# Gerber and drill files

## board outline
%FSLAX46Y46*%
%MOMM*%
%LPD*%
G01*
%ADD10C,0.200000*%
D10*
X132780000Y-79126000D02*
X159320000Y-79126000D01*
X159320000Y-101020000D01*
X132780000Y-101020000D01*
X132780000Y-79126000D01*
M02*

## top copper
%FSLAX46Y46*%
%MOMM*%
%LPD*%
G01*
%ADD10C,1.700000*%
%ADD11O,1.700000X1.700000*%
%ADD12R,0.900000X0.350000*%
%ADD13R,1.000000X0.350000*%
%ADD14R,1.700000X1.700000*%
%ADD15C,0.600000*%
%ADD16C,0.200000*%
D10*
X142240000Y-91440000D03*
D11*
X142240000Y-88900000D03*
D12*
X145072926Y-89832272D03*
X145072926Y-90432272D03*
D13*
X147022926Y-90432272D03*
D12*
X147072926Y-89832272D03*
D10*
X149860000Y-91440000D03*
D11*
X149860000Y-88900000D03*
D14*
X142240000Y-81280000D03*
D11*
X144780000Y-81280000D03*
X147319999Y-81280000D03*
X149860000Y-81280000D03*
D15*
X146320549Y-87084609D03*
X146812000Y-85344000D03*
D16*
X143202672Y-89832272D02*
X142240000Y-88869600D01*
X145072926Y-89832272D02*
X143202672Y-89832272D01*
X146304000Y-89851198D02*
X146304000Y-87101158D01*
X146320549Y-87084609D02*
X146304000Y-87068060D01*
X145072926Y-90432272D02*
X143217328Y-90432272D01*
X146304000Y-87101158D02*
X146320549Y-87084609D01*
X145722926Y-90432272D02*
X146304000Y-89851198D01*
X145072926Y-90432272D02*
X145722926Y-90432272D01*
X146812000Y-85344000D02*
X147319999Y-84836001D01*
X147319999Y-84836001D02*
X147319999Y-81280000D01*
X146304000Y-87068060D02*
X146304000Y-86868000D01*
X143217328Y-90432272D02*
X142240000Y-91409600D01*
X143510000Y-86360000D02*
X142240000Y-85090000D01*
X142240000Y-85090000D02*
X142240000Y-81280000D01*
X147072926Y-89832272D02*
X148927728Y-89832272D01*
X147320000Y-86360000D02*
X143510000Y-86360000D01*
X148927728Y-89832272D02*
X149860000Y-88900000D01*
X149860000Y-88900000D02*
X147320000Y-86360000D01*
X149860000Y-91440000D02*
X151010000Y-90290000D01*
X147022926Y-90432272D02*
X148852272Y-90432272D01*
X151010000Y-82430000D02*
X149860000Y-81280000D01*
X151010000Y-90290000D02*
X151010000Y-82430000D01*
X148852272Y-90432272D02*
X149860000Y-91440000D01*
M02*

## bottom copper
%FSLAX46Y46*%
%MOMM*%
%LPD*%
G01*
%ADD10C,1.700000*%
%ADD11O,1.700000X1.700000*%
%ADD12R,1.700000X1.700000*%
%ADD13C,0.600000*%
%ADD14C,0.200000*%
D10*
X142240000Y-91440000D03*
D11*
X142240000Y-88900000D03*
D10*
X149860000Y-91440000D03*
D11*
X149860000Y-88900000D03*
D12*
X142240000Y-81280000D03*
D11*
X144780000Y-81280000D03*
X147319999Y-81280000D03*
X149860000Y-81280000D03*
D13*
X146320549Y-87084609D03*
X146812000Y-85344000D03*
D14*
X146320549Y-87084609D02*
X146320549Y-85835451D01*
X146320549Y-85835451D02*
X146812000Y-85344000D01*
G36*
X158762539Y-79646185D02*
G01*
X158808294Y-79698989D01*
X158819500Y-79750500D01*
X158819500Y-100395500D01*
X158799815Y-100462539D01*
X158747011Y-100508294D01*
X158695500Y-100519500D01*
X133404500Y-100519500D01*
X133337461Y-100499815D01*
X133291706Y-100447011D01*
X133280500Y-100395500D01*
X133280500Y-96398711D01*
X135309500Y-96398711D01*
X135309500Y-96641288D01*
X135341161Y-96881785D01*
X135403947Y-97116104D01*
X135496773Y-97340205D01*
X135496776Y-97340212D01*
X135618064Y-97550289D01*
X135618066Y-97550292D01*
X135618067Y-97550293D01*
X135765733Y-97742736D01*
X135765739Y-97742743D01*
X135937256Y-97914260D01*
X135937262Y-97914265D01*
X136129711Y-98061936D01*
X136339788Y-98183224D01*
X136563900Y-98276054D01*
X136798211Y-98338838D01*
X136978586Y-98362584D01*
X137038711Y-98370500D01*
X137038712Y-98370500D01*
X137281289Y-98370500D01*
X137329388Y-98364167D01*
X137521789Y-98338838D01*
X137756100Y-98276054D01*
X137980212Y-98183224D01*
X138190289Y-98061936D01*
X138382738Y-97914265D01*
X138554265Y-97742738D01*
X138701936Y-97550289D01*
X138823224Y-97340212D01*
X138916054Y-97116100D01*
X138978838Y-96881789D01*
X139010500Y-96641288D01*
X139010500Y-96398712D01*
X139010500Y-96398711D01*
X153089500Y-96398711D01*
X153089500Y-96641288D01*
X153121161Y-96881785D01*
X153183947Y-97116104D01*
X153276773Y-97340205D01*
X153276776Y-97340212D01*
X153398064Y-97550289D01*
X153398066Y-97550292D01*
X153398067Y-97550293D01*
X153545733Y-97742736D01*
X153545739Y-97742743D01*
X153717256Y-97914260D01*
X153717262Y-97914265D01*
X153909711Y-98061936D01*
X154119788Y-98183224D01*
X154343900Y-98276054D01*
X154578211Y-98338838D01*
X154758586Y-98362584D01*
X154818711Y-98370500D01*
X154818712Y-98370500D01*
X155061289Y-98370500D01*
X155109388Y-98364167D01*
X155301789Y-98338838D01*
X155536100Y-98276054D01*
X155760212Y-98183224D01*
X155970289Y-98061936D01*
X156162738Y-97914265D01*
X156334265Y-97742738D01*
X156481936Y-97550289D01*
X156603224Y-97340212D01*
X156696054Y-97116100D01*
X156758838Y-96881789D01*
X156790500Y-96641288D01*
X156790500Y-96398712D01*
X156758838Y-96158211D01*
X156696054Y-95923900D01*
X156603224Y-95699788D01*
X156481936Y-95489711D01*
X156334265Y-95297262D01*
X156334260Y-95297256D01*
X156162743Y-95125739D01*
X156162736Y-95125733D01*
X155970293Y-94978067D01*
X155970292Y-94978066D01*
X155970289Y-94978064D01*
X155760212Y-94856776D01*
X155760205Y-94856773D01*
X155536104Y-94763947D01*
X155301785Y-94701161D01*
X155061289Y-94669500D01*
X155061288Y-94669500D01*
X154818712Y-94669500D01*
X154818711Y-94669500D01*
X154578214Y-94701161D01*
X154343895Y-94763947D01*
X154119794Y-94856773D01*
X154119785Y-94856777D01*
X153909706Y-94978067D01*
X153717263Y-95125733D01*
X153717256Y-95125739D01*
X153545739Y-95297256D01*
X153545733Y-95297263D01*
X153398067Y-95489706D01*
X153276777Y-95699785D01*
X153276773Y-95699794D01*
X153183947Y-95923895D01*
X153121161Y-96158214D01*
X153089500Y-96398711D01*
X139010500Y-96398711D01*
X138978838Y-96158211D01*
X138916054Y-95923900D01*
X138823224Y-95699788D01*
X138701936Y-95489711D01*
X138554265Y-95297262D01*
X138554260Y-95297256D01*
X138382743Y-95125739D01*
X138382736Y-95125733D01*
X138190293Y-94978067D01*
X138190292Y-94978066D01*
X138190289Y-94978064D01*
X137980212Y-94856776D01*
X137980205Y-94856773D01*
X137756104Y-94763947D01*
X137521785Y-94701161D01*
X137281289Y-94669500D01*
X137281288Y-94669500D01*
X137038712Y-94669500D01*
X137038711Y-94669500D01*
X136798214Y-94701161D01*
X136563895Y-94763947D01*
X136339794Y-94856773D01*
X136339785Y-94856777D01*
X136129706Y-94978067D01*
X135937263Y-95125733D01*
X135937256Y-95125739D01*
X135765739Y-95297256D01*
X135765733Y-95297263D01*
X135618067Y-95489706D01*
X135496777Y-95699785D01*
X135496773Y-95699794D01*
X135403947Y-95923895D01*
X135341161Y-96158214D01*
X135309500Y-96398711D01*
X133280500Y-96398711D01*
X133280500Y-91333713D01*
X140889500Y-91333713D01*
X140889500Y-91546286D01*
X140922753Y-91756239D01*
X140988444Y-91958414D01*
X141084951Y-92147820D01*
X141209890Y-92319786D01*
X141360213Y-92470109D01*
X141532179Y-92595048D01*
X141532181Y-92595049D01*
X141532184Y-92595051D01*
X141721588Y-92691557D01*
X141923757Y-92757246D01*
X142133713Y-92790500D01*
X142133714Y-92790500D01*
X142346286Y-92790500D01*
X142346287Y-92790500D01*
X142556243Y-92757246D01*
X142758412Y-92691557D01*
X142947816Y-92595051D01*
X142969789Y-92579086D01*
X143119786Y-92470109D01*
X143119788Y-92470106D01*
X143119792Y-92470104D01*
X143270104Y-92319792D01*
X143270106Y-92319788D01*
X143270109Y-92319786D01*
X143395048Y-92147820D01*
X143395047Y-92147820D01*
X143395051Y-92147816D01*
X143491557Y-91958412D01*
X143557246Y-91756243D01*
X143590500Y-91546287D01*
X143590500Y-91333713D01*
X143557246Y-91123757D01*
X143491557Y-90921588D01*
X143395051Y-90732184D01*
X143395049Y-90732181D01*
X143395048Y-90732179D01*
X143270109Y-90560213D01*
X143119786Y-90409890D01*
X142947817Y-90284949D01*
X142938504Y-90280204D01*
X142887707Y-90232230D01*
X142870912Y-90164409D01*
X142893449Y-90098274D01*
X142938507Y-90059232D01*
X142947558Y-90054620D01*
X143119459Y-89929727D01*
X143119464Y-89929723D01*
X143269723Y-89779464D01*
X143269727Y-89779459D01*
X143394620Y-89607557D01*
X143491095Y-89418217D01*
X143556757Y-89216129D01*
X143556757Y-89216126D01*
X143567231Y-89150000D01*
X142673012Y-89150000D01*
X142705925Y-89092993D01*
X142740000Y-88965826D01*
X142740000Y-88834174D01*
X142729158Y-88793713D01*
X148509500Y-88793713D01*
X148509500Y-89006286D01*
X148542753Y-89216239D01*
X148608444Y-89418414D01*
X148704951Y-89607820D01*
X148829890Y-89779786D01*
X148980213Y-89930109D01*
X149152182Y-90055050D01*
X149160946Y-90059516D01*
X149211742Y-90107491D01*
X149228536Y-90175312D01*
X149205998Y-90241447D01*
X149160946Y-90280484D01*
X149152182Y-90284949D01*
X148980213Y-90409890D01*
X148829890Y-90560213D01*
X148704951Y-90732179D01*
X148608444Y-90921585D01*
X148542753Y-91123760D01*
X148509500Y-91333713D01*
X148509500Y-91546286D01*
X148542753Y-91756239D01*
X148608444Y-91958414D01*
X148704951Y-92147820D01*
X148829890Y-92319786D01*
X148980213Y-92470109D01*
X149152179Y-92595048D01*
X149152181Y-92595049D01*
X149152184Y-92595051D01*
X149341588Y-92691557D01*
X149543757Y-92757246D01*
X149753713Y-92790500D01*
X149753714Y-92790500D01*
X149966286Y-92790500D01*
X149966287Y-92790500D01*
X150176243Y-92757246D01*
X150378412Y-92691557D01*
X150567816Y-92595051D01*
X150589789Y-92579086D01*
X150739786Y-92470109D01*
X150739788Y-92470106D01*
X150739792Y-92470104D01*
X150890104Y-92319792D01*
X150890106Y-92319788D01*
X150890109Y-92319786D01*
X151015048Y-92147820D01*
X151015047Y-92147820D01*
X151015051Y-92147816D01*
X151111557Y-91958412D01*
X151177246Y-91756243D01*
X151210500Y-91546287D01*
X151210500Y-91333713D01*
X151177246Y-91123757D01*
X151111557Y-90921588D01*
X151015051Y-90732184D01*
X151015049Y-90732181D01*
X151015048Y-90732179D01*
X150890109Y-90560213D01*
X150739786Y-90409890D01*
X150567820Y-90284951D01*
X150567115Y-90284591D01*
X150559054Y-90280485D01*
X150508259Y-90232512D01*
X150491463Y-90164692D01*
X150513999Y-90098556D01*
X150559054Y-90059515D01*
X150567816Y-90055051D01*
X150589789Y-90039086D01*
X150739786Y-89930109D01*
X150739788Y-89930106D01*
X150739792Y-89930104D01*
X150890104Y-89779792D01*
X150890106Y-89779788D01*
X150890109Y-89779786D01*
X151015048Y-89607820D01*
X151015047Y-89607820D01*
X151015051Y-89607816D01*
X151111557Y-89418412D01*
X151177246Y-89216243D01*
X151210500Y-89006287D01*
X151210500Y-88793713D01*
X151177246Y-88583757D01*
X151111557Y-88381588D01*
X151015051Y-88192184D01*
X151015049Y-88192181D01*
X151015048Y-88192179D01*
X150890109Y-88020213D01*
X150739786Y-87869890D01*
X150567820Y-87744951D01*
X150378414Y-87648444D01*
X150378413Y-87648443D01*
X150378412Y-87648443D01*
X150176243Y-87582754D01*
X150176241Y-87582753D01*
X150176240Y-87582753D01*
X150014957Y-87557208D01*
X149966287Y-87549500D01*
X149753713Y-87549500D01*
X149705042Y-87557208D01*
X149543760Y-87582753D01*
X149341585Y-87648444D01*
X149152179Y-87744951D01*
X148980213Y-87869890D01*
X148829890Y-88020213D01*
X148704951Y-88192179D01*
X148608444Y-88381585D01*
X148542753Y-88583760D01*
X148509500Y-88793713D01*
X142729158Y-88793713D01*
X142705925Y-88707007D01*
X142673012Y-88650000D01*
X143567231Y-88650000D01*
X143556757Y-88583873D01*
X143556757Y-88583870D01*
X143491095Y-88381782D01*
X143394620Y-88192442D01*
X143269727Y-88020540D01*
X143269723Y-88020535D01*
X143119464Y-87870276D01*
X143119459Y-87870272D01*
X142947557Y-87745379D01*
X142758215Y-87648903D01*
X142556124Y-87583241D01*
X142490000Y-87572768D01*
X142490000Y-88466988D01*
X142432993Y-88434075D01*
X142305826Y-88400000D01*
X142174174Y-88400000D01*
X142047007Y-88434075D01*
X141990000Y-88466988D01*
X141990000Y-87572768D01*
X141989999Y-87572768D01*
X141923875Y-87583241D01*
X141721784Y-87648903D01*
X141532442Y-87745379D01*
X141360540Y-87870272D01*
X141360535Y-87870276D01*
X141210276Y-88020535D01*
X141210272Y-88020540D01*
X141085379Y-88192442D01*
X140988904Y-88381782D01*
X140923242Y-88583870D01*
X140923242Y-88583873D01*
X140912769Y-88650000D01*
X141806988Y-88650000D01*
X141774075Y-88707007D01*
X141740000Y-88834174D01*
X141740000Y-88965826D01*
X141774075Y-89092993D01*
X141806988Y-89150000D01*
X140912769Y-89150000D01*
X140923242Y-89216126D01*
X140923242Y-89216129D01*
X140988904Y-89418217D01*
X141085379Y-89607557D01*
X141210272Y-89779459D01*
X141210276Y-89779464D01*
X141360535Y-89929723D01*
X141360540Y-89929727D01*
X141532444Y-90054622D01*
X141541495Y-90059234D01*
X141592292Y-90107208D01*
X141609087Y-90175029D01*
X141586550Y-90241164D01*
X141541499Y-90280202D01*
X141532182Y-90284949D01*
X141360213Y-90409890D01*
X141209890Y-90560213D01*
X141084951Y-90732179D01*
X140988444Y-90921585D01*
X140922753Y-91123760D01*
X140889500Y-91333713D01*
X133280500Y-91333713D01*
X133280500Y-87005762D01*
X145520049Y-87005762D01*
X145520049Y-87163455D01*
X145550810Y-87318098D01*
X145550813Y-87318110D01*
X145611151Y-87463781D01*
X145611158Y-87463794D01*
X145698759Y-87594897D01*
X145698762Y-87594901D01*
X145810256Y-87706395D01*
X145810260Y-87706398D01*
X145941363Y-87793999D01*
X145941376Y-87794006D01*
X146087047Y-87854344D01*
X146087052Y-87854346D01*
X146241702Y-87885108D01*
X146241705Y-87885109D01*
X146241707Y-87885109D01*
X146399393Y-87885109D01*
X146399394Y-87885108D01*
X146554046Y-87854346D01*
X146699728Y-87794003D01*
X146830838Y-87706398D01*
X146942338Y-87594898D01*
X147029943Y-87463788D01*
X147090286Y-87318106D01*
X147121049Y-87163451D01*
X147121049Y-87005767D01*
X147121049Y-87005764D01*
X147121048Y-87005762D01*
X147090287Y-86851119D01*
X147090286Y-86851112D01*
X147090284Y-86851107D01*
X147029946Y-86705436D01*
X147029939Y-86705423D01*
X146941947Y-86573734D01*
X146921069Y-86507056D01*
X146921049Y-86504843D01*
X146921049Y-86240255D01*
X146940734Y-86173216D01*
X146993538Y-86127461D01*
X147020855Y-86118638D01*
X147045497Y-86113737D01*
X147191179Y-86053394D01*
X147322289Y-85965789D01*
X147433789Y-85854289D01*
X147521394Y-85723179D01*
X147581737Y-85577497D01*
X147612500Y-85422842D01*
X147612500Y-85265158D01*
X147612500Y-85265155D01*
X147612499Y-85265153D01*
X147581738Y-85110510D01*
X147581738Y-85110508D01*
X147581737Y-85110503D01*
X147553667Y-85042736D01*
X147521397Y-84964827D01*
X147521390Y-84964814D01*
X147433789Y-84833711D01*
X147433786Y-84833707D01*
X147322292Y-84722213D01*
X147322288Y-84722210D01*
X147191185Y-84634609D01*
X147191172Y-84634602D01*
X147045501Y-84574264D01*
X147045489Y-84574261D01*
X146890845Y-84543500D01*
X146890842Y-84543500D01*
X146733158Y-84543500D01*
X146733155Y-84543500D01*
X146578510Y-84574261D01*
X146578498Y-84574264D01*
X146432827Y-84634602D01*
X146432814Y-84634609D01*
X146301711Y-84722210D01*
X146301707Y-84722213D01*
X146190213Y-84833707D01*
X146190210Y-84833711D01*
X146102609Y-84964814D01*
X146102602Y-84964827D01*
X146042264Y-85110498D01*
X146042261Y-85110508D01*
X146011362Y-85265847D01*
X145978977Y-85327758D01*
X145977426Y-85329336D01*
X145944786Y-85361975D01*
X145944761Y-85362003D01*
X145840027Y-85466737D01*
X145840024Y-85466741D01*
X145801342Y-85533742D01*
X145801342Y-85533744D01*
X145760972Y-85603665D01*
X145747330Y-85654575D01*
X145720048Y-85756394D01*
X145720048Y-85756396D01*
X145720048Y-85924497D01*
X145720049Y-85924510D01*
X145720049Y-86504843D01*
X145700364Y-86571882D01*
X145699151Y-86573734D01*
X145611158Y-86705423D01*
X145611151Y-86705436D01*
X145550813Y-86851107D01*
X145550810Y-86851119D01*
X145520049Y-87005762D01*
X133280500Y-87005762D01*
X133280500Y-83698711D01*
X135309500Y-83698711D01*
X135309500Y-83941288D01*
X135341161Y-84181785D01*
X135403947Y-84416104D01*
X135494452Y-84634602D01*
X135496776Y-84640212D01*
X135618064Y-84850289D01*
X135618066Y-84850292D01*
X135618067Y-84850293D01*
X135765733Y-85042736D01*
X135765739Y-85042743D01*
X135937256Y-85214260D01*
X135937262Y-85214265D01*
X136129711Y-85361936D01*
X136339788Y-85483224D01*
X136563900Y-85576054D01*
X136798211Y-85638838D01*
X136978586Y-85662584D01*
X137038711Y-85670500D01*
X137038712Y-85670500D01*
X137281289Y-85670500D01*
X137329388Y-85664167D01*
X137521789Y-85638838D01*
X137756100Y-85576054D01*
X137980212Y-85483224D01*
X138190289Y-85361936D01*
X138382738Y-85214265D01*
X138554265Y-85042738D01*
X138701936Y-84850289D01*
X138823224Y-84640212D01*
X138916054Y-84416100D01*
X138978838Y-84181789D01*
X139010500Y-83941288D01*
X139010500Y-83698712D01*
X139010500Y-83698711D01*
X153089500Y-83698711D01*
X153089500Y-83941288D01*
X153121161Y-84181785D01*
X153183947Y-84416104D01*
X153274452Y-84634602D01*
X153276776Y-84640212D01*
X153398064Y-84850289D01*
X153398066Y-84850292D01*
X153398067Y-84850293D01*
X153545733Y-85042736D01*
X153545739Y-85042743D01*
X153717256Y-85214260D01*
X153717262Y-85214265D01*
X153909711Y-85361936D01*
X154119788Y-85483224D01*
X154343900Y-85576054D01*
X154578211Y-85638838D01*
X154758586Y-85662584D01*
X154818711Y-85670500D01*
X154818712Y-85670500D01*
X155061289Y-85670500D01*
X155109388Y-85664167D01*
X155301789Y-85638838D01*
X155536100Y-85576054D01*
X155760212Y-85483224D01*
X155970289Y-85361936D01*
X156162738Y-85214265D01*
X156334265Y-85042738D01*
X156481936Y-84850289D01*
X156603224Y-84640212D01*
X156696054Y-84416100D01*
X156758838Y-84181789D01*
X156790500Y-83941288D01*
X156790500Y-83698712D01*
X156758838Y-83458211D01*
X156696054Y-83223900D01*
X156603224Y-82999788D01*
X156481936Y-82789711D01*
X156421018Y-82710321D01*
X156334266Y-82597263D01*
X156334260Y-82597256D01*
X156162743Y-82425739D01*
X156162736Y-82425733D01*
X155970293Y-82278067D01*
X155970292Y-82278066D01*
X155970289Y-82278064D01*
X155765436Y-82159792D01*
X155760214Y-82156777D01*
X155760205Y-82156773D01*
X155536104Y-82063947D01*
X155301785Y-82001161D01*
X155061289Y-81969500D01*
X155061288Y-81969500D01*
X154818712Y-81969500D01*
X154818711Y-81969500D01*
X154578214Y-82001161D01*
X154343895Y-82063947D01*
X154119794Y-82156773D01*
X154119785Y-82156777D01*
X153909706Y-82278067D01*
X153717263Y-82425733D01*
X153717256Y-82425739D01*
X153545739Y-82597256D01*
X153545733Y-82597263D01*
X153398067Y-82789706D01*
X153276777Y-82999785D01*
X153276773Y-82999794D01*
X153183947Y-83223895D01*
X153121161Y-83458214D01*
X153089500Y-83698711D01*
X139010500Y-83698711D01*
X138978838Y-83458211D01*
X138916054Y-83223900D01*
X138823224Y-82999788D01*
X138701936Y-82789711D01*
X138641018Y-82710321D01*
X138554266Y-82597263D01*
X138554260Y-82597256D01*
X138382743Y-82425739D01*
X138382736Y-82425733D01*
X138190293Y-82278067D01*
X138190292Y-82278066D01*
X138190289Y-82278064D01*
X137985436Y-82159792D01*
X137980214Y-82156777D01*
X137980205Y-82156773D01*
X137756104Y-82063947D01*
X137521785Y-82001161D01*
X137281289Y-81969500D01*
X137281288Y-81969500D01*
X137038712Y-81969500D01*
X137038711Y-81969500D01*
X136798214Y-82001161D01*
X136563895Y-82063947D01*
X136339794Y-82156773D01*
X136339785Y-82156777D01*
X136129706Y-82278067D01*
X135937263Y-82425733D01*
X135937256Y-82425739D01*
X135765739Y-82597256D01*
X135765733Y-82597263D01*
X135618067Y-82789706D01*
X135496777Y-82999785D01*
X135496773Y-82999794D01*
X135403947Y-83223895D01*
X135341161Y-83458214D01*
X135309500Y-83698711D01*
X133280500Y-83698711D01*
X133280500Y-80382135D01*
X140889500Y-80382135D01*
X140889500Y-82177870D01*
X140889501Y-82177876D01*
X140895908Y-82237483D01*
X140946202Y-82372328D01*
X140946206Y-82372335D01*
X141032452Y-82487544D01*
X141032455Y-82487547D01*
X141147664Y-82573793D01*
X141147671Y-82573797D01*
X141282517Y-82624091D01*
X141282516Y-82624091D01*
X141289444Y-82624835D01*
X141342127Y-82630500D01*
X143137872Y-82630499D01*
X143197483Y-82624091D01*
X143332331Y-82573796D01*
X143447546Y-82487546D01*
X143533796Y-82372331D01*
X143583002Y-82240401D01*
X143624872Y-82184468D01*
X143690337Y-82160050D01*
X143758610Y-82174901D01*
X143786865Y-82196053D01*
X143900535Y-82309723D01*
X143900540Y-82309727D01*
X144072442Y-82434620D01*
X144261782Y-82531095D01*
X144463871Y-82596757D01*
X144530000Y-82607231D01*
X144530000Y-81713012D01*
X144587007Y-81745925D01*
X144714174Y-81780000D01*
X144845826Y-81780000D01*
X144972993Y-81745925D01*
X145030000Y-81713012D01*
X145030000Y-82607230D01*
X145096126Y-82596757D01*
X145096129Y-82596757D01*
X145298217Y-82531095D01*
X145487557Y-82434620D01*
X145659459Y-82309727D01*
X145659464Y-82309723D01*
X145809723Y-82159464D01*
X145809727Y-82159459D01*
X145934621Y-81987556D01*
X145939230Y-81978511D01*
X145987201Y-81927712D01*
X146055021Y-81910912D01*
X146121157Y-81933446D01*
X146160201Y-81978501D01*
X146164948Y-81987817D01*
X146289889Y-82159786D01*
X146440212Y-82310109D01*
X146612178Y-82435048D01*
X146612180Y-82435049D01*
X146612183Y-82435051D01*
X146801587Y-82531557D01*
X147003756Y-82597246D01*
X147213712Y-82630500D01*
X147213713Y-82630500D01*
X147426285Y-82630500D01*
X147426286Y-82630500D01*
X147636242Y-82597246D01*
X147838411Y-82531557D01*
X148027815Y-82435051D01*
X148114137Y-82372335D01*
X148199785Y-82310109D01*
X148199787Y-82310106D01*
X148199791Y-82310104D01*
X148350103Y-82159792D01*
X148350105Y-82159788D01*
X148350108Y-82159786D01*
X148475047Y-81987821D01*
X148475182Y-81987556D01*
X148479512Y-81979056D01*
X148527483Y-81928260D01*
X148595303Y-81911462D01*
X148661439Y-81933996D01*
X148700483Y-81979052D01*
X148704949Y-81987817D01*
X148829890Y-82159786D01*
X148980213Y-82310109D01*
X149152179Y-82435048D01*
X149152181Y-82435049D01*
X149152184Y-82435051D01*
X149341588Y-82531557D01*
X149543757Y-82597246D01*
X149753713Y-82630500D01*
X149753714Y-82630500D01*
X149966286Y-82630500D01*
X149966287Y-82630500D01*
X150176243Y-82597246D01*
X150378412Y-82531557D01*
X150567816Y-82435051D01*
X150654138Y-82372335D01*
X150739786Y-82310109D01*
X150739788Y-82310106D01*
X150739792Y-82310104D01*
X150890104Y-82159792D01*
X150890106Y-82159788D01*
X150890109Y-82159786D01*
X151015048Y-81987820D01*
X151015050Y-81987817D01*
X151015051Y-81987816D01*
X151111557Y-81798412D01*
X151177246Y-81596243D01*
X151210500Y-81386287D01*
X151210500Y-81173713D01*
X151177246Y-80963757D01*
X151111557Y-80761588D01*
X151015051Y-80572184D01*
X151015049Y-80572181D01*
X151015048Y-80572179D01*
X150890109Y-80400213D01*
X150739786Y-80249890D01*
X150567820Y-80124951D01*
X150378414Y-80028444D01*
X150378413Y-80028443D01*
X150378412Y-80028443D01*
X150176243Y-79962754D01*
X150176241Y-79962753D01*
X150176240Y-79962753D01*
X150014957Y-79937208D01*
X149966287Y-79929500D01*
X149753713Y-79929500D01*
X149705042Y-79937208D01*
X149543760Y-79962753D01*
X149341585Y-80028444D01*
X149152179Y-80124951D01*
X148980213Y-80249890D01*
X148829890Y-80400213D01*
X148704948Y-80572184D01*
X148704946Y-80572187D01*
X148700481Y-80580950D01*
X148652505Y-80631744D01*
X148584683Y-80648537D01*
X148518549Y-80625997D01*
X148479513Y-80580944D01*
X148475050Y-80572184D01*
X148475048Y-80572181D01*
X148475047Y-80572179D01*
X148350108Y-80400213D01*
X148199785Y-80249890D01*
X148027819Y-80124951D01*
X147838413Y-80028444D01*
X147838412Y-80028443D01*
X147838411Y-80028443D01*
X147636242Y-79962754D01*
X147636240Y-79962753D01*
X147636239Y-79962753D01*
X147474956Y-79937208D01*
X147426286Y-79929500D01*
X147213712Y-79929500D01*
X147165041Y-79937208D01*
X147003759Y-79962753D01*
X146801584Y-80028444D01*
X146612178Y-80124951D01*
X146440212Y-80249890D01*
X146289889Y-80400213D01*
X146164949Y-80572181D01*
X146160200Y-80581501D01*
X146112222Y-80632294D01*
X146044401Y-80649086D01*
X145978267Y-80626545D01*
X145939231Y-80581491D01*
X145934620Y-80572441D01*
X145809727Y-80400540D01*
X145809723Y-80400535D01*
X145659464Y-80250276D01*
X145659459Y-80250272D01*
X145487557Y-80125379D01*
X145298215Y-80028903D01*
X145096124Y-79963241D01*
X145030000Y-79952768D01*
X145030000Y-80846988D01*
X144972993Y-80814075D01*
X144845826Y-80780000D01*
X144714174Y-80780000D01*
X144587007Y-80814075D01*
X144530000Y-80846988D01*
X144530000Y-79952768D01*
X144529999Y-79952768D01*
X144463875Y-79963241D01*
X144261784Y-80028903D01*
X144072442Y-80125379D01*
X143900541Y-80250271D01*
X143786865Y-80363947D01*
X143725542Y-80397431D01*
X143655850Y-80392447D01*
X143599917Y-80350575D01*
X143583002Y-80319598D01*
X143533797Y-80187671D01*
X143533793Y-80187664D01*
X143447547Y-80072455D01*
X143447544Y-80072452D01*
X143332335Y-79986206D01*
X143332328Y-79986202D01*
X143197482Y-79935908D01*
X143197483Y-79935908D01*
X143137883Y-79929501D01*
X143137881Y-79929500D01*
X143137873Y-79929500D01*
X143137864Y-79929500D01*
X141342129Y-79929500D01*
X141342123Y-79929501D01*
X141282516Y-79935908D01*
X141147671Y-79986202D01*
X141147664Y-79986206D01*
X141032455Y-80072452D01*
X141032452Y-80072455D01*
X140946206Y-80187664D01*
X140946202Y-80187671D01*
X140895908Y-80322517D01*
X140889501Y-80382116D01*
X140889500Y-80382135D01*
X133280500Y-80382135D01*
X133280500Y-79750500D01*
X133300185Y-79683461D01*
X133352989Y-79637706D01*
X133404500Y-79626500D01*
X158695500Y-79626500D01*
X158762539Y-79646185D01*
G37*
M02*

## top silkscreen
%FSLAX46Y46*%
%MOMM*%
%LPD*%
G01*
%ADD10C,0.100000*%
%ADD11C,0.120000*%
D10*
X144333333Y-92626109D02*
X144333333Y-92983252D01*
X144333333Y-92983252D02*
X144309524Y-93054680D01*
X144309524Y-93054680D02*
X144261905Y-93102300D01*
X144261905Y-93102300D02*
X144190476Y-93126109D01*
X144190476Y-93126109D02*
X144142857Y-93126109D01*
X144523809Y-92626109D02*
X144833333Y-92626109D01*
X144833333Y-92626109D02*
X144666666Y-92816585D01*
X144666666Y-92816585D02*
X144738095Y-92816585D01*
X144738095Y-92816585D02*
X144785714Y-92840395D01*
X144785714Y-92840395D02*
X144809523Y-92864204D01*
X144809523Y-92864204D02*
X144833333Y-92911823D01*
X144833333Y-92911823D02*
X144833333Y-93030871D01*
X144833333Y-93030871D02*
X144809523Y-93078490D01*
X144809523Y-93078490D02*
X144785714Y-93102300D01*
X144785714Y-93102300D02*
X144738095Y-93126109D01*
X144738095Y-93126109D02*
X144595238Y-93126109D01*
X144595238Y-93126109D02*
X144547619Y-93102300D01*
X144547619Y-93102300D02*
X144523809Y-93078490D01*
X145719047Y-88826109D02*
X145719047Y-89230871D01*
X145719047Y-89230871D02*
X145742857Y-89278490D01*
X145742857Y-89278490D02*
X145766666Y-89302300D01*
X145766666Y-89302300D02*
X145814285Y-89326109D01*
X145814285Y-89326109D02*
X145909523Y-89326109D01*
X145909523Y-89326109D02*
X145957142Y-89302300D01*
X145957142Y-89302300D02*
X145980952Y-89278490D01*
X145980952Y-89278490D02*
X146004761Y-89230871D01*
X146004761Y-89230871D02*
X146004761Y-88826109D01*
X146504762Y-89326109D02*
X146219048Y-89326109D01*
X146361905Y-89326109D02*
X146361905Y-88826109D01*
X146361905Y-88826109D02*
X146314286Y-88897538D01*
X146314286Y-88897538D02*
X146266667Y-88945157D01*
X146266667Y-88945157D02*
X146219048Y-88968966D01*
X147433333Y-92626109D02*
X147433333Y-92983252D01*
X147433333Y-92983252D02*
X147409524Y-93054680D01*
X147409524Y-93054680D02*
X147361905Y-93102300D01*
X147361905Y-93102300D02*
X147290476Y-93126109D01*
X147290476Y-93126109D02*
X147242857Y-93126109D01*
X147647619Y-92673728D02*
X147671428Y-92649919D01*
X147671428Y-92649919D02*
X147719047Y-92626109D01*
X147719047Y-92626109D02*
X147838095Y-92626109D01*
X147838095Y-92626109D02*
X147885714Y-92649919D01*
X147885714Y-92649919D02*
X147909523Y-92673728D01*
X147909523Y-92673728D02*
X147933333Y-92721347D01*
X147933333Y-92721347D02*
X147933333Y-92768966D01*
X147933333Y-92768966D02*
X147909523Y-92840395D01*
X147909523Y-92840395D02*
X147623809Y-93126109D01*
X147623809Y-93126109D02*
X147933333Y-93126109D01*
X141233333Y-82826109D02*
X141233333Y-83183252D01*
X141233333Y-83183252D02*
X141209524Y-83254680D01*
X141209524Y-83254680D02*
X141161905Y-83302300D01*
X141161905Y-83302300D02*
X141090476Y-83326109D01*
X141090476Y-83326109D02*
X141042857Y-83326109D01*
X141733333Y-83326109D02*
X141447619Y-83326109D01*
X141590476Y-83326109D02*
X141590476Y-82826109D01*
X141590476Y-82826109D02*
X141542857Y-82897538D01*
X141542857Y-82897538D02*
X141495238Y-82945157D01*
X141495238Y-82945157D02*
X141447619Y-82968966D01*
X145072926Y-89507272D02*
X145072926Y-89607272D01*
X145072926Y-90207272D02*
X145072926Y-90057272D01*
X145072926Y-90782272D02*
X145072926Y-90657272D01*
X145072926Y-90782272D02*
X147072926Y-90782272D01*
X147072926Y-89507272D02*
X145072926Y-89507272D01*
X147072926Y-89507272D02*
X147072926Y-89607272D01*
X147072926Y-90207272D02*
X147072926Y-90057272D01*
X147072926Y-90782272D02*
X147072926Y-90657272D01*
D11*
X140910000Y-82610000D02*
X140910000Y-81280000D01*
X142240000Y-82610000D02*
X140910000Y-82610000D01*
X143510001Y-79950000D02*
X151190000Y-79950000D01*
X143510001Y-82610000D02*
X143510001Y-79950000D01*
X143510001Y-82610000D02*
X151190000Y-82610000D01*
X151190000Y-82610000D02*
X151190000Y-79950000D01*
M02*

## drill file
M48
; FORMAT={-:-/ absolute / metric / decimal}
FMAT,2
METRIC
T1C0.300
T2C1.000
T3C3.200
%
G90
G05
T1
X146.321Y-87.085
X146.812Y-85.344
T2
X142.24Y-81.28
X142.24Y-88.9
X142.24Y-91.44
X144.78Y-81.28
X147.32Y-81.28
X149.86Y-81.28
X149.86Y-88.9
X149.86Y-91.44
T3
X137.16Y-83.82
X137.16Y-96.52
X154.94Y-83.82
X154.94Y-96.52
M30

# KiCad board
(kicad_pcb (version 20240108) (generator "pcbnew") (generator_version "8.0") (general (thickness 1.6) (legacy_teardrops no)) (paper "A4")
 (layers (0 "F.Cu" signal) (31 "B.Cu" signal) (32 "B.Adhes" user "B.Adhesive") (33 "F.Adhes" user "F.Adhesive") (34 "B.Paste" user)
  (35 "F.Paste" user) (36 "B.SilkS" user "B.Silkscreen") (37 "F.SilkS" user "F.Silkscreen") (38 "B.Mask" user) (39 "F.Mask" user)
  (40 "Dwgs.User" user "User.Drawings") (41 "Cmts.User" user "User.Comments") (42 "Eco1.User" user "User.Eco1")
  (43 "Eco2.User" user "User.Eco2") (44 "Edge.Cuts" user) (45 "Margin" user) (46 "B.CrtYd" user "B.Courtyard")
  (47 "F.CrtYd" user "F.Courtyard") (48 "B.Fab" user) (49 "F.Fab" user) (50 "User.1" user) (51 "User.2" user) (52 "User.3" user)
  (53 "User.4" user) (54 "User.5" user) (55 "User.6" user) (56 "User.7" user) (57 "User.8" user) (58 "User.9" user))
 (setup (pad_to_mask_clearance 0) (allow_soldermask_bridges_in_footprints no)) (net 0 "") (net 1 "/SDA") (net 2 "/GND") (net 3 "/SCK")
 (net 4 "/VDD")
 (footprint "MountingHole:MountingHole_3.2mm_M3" (layer "F.Cu") (at 137.16 83.82)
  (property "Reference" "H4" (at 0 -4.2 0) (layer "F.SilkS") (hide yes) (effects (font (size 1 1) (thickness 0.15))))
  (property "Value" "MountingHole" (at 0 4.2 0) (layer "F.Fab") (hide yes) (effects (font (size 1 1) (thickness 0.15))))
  (pad "" np_thru_hole circle (at 0 0) (size 3.2 3.2) (drill 3.2) (layers "*.Cu" "*.Mask")))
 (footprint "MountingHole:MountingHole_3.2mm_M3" (layer "F.Cu") (at 154.94 83.82)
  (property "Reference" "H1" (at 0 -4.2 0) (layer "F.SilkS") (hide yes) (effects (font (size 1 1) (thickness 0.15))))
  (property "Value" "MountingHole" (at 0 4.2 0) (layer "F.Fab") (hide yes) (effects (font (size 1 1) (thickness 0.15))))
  (pad "" np_thru_hole circle (at 0 0) (size 3.2 3.2) (drill 3.2) (layers "*.Cu" "*.Mask")))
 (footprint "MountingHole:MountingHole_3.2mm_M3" (layer "F.Cu") (at 137.16 96.52)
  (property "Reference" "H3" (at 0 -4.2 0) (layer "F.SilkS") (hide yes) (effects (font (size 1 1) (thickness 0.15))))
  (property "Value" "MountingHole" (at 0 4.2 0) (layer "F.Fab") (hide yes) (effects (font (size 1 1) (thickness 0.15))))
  (pad "" np_thru_hole circle (at 0 0) (size 3.2 3.2) (drill 3.2) (layers "*.Cu" "*.Mask")))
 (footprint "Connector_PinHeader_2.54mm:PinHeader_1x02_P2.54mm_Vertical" (layer "F.Cu") (at 142.24 91.44 180)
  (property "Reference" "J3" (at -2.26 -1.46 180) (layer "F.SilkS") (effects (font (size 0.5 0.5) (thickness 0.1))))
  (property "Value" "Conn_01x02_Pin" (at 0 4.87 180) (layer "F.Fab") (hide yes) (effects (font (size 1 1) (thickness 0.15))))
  (pad "1" thru_hole circle (at 0 0 180) (size 1.7 1.7) (drill 1) (layers "*.Cu" "*.Mask") (remove_unused_layers no) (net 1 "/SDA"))
  (pad "2" thru_hole oval (at 0 2.54 180) (size 1.7 1.7) (drill 1) (layers "*.Cu" "*.Mask") (remove_unused_layers no) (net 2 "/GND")))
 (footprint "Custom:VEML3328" (layer "F.Cu") (at 146.172926 90.732272)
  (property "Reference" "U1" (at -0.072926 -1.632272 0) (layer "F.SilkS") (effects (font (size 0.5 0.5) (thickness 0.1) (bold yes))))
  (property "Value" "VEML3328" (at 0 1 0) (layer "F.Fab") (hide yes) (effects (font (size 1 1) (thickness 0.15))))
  (fp_line (start -1.1 -1.225) (end -1.1 -1.125) (stroke (width 0.1) (type default)) (layer "F.SilkS"))
  (fp_line (start -1.1 -0.525) (end -1.1 -0.675) (stroke (width 0.1) (type default)) (layer "F.SilkS"))
  (fp_line (start -1.1 0.05) (end -1.1 -0.075) (stroke (width 0.1) (type default)) (layer "F.SilkS"))
  (fp_line (start -1.1 0.05) (end 0.9 0.05) (stroke (width 0.1) (type default)) (layer "F.SilkS"))
  (fp_line (start 0.9 -1.225) (end -1.1 -1.225) (stroke (width 0.1) (type default)) (layer "F.SilkS"))
  (fp_line (start 0.9 -1.225) (end 0.9 -1.125) (stroke (width 0.1) (type default)) (layer "F.SilkS"))
  (fp_line (start 0.9 -0.525) (end 0.9 -0.675) (stroke (width 0.1) (type default)) (layer "F.SilkS"))
  (fp_line (start 0.9 0.05) (end 0.9 -0.075) (stroke (width 0.1) (type default)) (layer "F.SilkS"))
  (pad "1" smd rect (at -1.1 -0.9) (size 0.9 0.35) (layers "F.Cu" "F.Paste" "F.Mask") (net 2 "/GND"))
  (pad "2" smd rect (at -1.1 -0.3) (size 0.9 0.35) (layers "F.Cu" "F.Paste" "F.Mask") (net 1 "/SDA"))
  (pad "3" smd rect (at 0.85 -0.3) (size 1 0.35) (layers "F.Cu" "F.Paste" "F.Mask") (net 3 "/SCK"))
  (pad "4" smd rect (at 0.9 -0.9) (size 0.9 0.35) (layers "F.Cu" "F.Paste" "F.Mask") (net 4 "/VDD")))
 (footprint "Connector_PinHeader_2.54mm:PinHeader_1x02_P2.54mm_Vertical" (layer "F.Cu") (at 149.86 91.44 180)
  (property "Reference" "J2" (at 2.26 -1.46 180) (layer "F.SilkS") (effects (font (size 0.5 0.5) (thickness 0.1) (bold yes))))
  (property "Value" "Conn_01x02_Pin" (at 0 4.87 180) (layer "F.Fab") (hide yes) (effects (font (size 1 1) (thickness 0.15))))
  (pad "1" thru_hole circle (at 0 0 180) (size 1.7 1.7) (drill 1) (layers "*.Cu" "*.Mask") (remove_unused_layers no) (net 3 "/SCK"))
  (pad "2" thru_hole oval (at 0 2.54 180) (size 1.7 1.7) (drill 1) (layers "*.Cu" "*.Mask") (remove_unused_layers no) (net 4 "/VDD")))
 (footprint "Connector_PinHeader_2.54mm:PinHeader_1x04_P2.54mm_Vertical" (layer "F.Cu") (at 142.24 81.28 90)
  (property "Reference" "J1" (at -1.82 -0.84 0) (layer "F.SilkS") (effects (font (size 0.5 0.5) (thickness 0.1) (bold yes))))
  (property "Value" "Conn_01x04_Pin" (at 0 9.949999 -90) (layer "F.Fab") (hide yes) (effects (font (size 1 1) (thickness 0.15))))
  (fp_line (start -1.33 -1.33) (end 0 -1.33) (stroke (width 0.12) (type solid)) (layer "F.SilkS"))
  (fp_line (start -1.33 0) (end -1.33 -1.33) (stroke (width 0.12) (type solid)) (layer "F.SilkS"))
  (fp_line (start 1.33 1.270001) (end 1.33 8.95) (stroke (width 0.12) (type solid)) (layer "F.SilkS"))
  (fp_line (start -1.33 1.270001) (end 1.33 1.270001) (stroke (width 0.12) (type solid)) (layer "F.SilkS"))
  (fp_line (start -1.33 1.270001) (end -1.33 8.95) (stroke (width 0.12) (type solid)) (layer "F.SilkS"))
  (fp_line (start -1.33 8.95) (end 1.33 8.95) (stroke (width 0.12) (type solid)) (layer "F.SilkS"))
  (pad "1" thru_hole rect (at 0 0 90) (size 1.7 1.7) (drill 1) (layers "*.Cu" "*.Mask") (remove_unused_layers no) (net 4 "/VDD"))
  (pad "2" thru_hole oval (at 0 2.54 90) (size 1.7 1.7) (drill 1) (layers "*.Cu" "*.Mask") (remove_unused_layers no) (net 2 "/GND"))
  (pad "3" thru_hole oval (at 0 5.079999 90) (size 1.7 1.7) (drill 1) (layers "*.Cu" "*.Mask") (remove_unused_layers no) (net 1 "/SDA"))
  (pad "4" thru_hole oval (at 0 7.62 90) (size 1.7 1.7) (drill 1) (layers "*.Cu" "*.Mask") (remove_unused_layers no) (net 3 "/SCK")))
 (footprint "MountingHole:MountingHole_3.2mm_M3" (layer "F.Cu") (at 154.94 96.52)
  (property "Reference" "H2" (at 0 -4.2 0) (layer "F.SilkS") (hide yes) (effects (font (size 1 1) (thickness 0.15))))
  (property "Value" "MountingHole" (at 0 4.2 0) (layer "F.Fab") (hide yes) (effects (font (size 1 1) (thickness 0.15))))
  (pad "" np_thru_hole circle (at 0 0) (size 3.2 3.2) (drill 3.2) (layers "*.Cu" "*.Mask")))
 (gr_rect (start 132.78 79.126) (end 159.32 101.02) (stroke (width 0.2) (type default)) (fill none) (layer "Edge.Cuts"))
 (segment (start 143.202672 89.832272) (end 142.24 88.8696) (width 0.2) (layer "F.Cu") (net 2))
 (segment (start 145.072926 89.832272) (end 143.202672 89.832272) (width 0.2) (layer "F.Cu") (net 2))
 (segment (start 146.304 89.851198) (end 146.304 87.101158) (width 0.2) (layer "F.Cu") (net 1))
 (segment (start 146.320549 87.084609) (end 146.304 87.06806) (width 0.2) (layer "F.Cu") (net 1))
 (segment (start 145.072926 90.432272) (end 143.217328 90.432272) (width 0.2) (layer "F.Cu") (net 1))
 (segment (start 146.304 87.101158) (end 146.320549 87.084609) (width 0.2) (layer "F.Cu") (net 1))
 (segment (start 145.722926 90.432272) (end 146.304 89.851198) (width 0.2) (layer "F.Cu") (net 1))
 (segment (start 145.072926 90.432272) (end 145.722926 90.432272) (width 0.2) (layer "F.Cu") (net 1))
 (segment (start 146.812 85.344) (end 147.319999 84.836001) (width 0.2) (layer "F.Cu") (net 1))
 (segment (start 147.319999 84.836001) (end 147.319999 81.28) (width 0.2) (layer "F.Cu") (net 1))
 (segment (start 146.304 87.06806) (end 146.304 86.868) (width 0.2) (layer "F.Cu") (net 1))
 (segment (start 143.217328 90.432272) (end 142.24 91.4096) (width 0.2) (layer "F.Cu") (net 1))
 (via (at 146.320549 87.084609) (size 0.6) (drill 0.3) (layers "F.Cu" "B.Cu") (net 1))
 (via (at 146.812 85.344) (size 0.6) (drill 0.3) (layers "F.Cu" "B.Cu") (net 1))
 (segment (start 146.320549 87.084609) (end 146.320549 85.835451) (width 0.2) (layer "B.Cu") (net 1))
 (segment (start 146.320549 85.835451) (end 146.812 85.344) (width 0.2) (layer "B.Cu") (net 1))
 (segment (start 143.51 86.36) (end 142.24 85.09) (width 0.2) (layer "F.Cu") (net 4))
 (segment (start 142.24 85.09) (end 142.24 81.28) (width 0.2) (layer "F.Cu") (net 4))
 (segment (start 147.072926 89.832272) (end 148.927728 89.832272) (width 0.2) (layer "F.Cu") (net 4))
 (segment (start 147.32 86.36) (end 143.51 86.36) (width 0.2) (layer "F.Cu") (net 4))
 (segment (start 148.927728 89.832272) (end 149.86 88.9) (width 0.2) (layer "F.Cu") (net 4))
 (segment (start 149.86 88.9) (end 147.32 86.36) (width 0.2) (layer "F.Cu") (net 4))
 (segment (start 149.86 91.44) (end 151.01 90.29) (width 0.2) (layer "F.Cu") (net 3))
 (segment (start 147.022926 90.432272) (end 148.852272 90.432272) (width 0.2) (layer "F.Cu") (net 3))
 (segment (start 151.01 82.43) (end 149.86 81.28) (width 0.2) (layer "F.Cu") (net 3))
 (segment (start 151.01 90.29) (end 151.01 82.43) (width 0.2) (layer "F.Cu") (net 3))
 (segment (start 148.852272 90.432272) (end 149.86 91.44) (width 0.2) (layer "F.Cu") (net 3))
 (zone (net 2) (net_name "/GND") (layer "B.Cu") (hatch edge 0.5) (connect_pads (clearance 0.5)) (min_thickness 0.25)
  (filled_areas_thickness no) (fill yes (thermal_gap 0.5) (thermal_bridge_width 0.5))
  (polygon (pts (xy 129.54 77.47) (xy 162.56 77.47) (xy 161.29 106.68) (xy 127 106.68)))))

